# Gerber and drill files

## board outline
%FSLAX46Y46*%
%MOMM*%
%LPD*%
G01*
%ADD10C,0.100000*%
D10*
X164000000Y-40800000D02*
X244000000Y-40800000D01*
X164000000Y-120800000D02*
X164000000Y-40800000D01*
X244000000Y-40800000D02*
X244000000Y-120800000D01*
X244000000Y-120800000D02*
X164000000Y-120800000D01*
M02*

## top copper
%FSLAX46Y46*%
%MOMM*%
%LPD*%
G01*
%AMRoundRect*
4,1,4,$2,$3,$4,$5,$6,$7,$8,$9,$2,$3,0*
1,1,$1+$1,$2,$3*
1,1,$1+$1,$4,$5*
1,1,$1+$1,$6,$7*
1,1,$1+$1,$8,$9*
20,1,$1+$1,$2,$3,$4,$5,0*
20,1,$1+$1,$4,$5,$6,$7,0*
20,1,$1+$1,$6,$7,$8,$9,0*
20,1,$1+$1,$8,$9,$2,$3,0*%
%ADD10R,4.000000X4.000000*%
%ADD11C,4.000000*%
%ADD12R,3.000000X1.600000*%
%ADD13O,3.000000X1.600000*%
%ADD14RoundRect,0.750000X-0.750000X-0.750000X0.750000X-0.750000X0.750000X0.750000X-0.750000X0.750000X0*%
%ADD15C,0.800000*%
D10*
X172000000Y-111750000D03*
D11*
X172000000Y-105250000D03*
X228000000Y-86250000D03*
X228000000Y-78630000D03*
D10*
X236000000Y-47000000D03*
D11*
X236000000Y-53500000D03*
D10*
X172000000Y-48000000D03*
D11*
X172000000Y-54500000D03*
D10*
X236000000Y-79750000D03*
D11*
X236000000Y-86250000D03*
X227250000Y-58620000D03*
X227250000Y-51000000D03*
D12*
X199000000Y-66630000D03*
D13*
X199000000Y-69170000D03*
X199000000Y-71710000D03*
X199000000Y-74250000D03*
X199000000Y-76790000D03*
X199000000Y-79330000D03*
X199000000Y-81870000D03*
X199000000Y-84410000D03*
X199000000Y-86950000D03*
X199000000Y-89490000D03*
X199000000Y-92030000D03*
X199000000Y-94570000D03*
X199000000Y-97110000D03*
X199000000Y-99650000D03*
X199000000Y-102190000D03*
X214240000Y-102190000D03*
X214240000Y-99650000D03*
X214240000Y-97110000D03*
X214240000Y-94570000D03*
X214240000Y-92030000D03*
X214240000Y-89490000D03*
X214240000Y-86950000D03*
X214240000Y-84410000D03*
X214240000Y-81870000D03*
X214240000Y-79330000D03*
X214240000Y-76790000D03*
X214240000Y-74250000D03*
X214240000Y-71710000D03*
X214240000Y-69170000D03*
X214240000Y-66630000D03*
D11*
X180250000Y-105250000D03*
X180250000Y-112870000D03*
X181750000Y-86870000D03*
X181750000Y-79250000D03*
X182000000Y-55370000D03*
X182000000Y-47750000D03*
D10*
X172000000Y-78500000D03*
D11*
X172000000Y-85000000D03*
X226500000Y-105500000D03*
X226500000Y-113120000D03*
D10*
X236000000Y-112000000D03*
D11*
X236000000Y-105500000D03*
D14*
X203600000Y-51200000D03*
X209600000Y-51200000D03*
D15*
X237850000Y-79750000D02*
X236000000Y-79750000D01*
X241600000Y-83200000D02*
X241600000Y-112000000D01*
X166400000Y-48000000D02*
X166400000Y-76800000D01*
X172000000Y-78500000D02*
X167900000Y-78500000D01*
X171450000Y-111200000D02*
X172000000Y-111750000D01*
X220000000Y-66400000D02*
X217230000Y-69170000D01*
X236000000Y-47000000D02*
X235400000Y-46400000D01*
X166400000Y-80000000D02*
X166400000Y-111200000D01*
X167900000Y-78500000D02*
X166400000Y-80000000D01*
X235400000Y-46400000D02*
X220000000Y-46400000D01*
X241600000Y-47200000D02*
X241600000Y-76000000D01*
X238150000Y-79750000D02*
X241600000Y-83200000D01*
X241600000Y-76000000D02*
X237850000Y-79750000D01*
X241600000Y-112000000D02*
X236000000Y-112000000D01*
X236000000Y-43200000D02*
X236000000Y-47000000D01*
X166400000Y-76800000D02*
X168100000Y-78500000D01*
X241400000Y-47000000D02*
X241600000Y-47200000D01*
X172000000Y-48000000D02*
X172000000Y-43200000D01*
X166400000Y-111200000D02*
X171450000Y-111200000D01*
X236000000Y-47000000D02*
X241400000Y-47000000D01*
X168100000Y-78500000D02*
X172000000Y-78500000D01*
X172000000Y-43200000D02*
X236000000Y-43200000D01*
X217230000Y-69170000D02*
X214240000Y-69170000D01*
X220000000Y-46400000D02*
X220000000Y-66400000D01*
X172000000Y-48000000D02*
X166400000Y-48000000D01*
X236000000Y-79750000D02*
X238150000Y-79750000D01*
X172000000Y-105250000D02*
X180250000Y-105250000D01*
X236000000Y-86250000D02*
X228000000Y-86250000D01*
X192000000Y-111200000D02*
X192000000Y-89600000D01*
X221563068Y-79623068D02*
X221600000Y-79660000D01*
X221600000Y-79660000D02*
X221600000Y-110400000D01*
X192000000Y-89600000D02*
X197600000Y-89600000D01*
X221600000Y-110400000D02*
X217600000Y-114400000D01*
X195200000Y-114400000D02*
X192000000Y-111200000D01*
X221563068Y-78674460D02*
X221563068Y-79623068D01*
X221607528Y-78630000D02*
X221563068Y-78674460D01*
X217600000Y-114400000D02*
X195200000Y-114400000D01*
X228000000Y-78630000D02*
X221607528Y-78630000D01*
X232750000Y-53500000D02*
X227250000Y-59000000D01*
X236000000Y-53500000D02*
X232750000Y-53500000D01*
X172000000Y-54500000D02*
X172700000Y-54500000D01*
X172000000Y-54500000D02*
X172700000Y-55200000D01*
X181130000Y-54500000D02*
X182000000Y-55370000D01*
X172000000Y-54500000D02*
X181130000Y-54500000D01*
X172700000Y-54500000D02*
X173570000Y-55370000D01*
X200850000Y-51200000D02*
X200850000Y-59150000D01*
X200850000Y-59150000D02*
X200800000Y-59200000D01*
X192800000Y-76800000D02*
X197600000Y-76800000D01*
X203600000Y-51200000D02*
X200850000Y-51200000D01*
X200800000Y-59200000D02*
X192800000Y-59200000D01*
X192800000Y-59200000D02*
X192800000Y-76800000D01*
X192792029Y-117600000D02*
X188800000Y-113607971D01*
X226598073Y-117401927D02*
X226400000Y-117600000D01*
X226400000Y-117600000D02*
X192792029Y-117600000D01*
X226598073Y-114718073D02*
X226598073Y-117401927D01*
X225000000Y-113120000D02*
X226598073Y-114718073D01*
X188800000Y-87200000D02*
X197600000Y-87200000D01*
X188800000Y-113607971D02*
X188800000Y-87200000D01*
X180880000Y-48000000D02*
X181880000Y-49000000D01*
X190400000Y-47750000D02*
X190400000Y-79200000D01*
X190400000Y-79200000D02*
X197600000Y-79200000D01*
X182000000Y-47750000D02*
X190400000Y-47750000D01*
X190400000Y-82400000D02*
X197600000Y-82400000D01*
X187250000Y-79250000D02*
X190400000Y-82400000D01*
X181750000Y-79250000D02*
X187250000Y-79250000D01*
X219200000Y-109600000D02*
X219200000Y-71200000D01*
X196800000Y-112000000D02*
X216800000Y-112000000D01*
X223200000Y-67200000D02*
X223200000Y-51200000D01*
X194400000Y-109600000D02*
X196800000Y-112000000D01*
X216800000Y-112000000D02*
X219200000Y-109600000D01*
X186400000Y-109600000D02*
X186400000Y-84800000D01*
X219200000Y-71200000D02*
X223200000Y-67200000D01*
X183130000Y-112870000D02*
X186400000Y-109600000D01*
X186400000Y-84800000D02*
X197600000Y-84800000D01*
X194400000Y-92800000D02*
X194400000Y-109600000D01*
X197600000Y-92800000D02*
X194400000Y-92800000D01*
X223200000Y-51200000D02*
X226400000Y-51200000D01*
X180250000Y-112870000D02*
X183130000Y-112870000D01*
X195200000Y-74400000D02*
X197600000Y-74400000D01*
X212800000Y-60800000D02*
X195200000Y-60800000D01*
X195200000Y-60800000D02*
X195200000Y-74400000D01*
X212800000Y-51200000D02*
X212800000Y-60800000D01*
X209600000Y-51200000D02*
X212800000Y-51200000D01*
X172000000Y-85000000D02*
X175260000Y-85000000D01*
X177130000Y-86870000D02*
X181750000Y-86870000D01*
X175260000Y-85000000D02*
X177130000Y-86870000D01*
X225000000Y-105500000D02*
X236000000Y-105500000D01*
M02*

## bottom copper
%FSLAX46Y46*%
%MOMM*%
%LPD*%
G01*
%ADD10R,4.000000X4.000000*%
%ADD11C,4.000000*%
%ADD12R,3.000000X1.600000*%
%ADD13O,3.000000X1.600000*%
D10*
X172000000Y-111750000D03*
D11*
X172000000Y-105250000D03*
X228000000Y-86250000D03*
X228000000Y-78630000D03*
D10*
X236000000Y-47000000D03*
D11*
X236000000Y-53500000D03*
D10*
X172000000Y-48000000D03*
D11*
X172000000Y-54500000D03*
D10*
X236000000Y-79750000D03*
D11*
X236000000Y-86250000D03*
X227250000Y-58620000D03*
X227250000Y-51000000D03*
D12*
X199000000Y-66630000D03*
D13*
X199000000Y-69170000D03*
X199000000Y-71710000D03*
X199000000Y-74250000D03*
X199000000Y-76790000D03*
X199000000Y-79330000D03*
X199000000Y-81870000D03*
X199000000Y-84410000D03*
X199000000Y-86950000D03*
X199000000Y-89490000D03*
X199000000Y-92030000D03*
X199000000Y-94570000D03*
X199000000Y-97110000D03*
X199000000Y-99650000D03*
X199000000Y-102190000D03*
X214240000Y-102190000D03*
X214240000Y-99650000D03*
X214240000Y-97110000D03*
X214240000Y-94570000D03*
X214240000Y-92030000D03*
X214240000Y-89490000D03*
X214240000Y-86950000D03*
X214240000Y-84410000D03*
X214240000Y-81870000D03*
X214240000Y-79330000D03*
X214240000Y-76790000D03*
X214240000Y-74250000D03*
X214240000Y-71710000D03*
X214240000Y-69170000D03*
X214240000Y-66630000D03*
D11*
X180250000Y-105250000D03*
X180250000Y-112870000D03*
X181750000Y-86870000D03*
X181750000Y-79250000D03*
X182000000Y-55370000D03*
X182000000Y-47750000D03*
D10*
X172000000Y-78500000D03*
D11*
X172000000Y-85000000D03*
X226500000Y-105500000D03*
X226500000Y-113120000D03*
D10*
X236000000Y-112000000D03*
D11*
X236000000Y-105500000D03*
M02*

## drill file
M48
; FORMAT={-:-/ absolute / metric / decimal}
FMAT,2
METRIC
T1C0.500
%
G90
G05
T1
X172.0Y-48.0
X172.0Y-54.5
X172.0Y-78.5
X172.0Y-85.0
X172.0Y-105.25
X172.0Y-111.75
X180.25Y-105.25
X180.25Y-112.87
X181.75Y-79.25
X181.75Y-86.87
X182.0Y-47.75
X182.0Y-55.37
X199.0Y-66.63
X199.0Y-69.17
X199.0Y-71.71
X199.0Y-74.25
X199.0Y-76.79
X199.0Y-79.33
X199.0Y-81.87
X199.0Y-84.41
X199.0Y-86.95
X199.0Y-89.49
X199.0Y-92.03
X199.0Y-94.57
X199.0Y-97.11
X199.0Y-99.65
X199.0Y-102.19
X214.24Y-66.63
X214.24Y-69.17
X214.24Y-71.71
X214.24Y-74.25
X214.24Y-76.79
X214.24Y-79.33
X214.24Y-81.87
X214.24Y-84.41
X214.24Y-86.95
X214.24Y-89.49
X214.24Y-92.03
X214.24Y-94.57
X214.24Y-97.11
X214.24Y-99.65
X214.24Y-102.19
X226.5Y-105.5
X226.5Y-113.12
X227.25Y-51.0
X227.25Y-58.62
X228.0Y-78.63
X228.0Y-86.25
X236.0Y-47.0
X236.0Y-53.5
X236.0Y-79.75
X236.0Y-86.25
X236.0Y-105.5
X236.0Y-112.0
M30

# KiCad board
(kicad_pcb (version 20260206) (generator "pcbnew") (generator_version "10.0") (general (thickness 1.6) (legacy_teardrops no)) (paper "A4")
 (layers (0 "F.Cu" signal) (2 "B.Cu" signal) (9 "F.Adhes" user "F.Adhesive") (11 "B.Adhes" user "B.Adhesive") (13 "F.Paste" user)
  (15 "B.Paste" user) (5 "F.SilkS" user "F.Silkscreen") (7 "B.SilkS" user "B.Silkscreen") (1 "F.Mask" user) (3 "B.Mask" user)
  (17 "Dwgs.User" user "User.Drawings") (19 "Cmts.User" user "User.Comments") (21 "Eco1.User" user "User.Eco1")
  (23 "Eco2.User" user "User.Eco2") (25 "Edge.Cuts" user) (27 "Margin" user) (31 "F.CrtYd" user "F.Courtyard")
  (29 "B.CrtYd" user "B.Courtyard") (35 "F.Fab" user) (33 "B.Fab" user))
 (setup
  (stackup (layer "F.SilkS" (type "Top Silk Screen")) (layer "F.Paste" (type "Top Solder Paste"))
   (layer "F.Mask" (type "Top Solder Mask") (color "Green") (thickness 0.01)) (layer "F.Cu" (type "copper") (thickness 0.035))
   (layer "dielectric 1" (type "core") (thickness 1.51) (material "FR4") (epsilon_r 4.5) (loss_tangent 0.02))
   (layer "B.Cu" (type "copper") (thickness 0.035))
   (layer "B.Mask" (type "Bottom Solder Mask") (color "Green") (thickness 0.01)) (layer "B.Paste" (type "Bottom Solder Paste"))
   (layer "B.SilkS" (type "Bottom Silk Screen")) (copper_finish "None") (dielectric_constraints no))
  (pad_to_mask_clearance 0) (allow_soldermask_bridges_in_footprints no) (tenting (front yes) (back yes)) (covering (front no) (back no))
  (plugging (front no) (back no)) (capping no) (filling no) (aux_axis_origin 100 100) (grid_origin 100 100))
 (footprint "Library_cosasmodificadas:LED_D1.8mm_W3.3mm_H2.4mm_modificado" (layer "F.Cu") (at 172 109.25 90)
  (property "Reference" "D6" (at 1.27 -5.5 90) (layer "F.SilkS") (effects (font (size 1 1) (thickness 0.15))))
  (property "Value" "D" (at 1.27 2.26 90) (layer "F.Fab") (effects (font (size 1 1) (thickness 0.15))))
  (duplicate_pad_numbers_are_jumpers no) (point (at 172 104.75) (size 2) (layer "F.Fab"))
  (pad "1" thru_hole rect (at -2.5 0 90) (size 4 4) (drill 0.5) (layers "*.Cu" "*.Mask") (remove_unused_layers no) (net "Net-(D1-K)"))
  (pad "2" thru_hole circle (at 4 0 90) (size 4 4) (drill 0.5) (layers "*.Cu" "*.Mask") (remove_unused_layers no) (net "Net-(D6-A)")))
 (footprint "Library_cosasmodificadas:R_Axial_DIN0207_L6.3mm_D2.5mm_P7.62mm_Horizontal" (layer "F.Cu") (at 228 86.25 90)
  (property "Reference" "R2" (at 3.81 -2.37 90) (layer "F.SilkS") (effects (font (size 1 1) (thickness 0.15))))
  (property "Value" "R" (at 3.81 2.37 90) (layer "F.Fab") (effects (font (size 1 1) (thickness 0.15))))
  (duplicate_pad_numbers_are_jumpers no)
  (pad "1" thru_hole circle (at 0 0 90) (size 4 4) (drill 0.5) (layers "*.Cu" "*.Mask") (remove_unused_layers no) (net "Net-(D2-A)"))
  (pad "2" thru_hole circle (at 7.62 0 90) (size 4 4) (drill 0.5) (layers "*.Cu" "*.Mask") (remove_unused_layers no) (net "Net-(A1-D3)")))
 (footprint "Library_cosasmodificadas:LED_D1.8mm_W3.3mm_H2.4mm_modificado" (layer "F.Cu") (at 236 49.5 -90)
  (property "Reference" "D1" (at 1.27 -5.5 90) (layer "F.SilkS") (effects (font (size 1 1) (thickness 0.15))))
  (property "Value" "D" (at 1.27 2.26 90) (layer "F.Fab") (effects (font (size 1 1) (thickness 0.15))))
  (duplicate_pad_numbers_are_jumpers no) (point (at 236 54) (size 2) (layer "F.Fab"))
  (pad "1" thru_hole rect (at -2.5 0 270) (size 4 4) (drill 0.5) (layers "*.Cu" "*.Mask") (remove_unused_layers no) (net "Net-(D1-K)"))
  (pad "2" thru_hole circle (at 4 0 270) (size 4 4) (drill 0.5) (layers "*.Cu" "*.Mask") (remove_unused_layers no) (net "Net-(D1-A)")))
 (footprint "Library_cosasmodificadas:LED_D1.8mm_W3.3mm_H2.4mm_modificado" (layer "F.Cu") (at 172 50.5 -90)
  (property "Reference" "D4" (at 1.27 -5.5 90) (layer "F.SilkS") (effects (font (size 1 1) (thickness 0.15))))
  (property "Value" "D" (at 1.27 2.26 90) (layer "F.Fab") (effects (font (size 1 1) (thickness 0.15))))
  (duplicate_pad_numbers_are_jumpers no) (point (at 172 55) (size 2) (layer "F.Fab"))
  (pad "1" thru_hole rect (at -2.5 0 270) (size 4 4) (drill 0.5) (layers "*.Cu" "*.Mask") (remove_unused_layers no) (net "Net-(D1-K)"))
  (pad "2" thru_hole circle (at 4 0 270) (size 4 4) (drill 0.5) (layers "*.Cu" "*.Mask") (remove_unused_layers no) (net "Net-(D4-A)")))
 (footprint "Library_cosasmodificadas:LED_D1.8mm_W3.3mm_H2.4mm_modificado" (layer "F.Cu") (at 236 82.25 -90)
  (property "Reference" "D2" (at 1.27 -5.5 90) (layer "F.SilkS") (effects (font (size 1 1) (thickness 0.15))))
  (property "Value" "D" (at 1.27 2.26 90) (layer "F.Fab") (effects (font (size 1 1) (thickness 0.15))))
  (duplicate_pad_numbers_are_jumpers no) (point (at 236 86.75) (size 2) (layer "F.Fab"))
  (pad "1" thru_hole rect (at -2.5 0 270) (size 4 4) (drill 0.5) (layers "*.Cu" "*.Mask") (remove_unused_layers no) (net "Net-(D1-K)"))
  (pad "2" thru_hole circle (at 4 0 270) (size 4 4) (drill 0.5) (layers "*.Cu" "*.Mask") (remove_unused_layers no) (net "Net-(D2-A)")))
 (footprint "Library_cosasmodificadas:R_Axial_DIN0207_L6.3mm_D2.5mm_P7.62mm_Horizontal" (layer "F.Cu") (at 227.25 58.62 90)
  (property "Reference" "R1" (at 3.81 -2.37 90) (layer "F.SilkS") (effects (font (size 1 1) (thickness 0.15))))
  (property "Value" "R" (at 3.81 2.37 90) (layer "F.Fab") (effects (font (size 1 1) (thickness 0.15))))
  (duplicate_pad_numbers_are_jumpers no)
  (pad "1" thru_hole circle (at 0 0 90) (size 4 4) (drill 0.5) (layers "*.Cu" "*.Mask") (remove_unused_layers no) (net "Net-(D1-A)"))
  (pad "2" thru_hole circle (at 7.62 0 90) (size 4 4) (drill 0.5) (layers "*.Cu" "*.Mask") (remove_unused_layers no) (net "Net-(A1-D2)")))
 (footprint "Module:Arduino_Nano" (layer "F.Cu") (at 199 66.63)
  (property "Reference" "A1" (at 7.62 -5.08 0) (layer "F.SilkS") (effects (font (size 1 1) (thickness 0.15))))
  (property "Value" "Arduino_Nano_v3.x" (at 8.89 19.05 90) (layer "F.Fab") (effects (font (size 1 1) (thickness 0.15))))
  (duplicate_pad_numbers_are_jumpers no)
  (pad "1" thru_hole rect (at 0 0) (size 3 1.6) (drill 0.5) (layers "*.Cu" "*.Mask") (remove_unused_layers no)
   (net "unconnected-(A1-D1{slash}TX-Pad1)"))
  (pad "2" thru_hole oval (at 0 2.54) (size 3 1.6) (drill 0.5) (layers "*.Cu" "*.Mask") (remove_unused_layers no)
   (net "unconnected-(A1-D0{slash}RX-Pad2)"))
  (pad "3" thru_hole oval (at 0 5.08) (size 3 1.6) (drill 0.5) (layers "*.Cu" "*.Mask") (remove_unused_layers no)
   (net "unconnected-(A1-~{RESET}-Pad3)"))
  (pad "4" thru_hole oval (at 0 7.62) (size 3 1.6) (drill 0.5) (layers "*.Cu" "*.Mask") (remove_unused_layers no) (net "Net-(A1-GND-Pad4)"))
  (pad "5" thru_hole oval (at 0 10.16) (size 3 1.6) (drill 0.5) (layers "*.Cu" "*.Mask") (remove_unused_layers no) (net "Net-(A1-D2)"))
  (pad "6" thru_hole oval (at 0 12.7) (size 3 1.6) (drill 0.5) (layers "*.Cu" "*.Mask") (remove_unused_layers no) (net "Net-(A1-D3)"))
  (pad "7" thru_hole oval (at 0 15.24) (size 3 1.6) (drill 0.5) (layers "*.Cu" "*.Mask") (remove_unused_layers no) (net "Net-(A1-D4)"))
  (pad "8" thru_hole oval (at 0 17.78) (size 3 1.6) (drill 0.5) (layers "*.Cu" "*.Mask") (remove_unused_layers no) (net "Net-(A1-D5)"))
  (pad "9" thru_hole oval (at 0 20.32) (size 3 1.6) (drill 0.5) (layers "*.Cu" "*.Mask") (remove_unused_layers no) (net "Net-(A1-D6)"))
  (pad "10" thru_hole oval (at 0 22.86) (size 3 1.6) (drill 0.5) (layers "*.Cu" "*.Mask") (remove_unused_layers no)
   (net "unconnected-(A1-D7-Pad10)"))
  (pad "11" thru_hole oval (at 0 25.4) (size 3 1.6) (drill 0.5) (layers "*.Cu" "*.Mask") (remove_unused_layers no) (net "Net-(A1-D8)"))
  (pad "12" thru_hole oval (at 0 27.94) (size 3 1.6) (drill 0.5) (layers "*.Cu" "*.Mask") (remove_unused_layers no)
   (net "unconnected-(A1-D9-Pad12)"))
  (pad "13" thru_hole oval (at 0 30.48) (size 3 1.6) (drill 0.5) (layers "*.Cu" "*.Mask") (remove_unused_layers no)
   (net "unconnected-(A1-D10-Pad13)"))
  (pad "14" thru_hole oval (at 0 33.02) (size 3 1.6) (drill 0.5) (layers "*.Cu" "*.Mask") (remove_unused_layers no)
   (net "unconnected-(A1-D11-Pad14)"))
  (pad "15" thru_hole oval (at 0 35.56) (size 3 1.6) (drill 0.5) (layers "*.Cu" "*.Mask") (remove_unused_layers no)
   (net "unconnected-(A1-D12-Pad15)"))
  (pad "16" thru_hole oval (at 15.24 35.56) (size 3 1.6) (drill 0.5) (layers "*.Cu" "*.Mask") (remove_unused_layers no) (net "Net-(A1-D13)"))
  (pad "17" thru_hole oval (at 15.24 33.02) (size 3 1.6) (drill 0.5) (layers "*.Cu" "*.Mask") (remove_unused_layers no)
   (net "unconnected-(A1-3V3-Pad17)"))
  (pad "18" thru_hole oval (at 15.24 30.48) (size 3 1.6) (drill 0.5) (layers "*.Cu" "*.Mask") (remove_unused_layers no)
   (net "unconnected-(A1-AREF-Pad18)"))
  (pad "19" thru_hole oval (at 15.24 27.94) (size 3 1.6) (drill 0.5) (layers "*.Cu" "*.Mask") (remove_unused_layers no)
   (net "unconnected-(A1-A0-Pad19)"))
  (pad "20" thru_hole oval (at 15.24 25.4) (size 3 1.6) (drill 0.5) (layers "*.Cu" "*.Mask") (remove_unused_layers no)
   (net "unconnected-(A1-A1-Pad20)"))
  (pad "21" thru_hole oval (at 15.24 22.86) (size 3 1.6) (drill 0.5) (layers "*.Cu" "*.Mask") (remove_unused_layers no)
   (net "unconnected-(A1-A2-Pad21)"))
  (pad "22" thru_hole oval (at 15.24 20.32) (size 3 1.6) (drill 0.5) (layers "*.Cu" "*.Mask") (remove_unused_layers no)
   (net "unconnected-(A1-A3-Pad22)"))
  (pad "23" thru_hole oval (at 15.24 17.78) (size 3 1.6) (drill 0.5) (layers "*.Cu" "*.Mask") (remove_unused_layers no)
   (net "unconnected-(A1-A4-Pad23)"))
  (pad "24" thru_hole oval (at 15.24 15.24) (size 3 1.6) (drill 0.5) (layers "*.Cu" "*.Mask") (remove_unused_layers no)
   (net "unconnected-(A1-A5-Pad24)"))
  (pad "25" thru_hole oval (at 15.24 12.7) (size 3 1.6) (drill 0.5) (layers "*.Cu" "*.Mask") (remove_unused_layers no)
   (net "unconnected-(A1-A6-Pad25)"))
  (pad "26" thru_hole oval (at 15.24 10.16) (size 3 1.6) (drill 0.5) (layers "*.Cu" "*.Mask") (remove_unused_layers no)
   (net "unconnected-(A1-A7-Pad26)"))
  (pad "27" thru_hole oval (at 15.24 7.62) (size 3 1.6) (drill 0.5) (layers "*.Cu" "*.Mask") (remove_unused_layers no)
   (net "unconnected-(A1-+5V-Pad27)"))
  (pad "28" thru_hole oval (at 15.24 5.08) (size 3 1.6) (drill 0.5) (layers "*.Cu" "*.Mask") (remove_unused_layers no)
   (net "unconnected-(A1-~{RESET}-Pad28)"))
  (pad "29" thru_hole oval (at 15.24 2.54) (size 3 1.6) (drill 0.5) (layers "*.Cu" "*.Mask") (remove_unused_layers no) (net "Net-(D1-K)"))
  (pad "30" thru_hole oval (at 15.24 0) (size 3 1.6) (drill 0.5) (layers "*.Cu" "*.Mask") (remove_unused_layers no)
   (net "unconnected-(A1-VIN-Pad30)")))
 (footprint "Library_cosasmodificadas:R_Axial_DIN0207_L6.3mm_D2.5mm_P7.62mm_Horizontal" (layer "F.Cu") (at 180.25 105.25 -90)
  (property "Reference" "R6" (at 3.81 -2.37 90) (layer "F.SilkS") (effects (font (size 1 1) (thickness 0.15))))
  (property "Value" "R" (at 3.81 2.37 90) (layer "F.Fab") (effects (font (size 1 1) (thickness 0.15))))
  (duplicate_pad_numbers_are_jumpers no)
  (pad "1" thru_hole circle (at 0 0 270) (size 4 4) (drill 0.5) (layers "*.Cu" "*.Mask") (remove_unused_layers no) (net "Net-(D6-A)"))
  (pad "2" thru_hole circle (at 7.62 0 270) (size 4 4) (drill 0.5) (layers "*.Cu" "*.Mask") (remove_unused_layers no) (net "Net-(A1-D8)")))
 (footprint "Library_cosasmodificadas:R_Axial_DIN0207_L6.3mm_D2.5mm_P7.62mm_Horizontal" (layer "F.Cu") (at 181.75 86.87 90)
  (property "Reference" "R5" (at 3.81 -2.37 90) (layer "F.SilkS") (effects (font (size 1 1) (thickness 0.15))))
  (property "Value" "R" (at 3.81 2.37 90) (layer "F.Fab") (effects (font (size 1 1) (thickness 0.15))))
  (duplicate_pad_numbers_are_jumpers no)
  (pad "1" thru_hole circle (at 0 0 90) (size 4 4) (drill 0.5) (layers "*.Cu" "*.Mask") (remove_unused_layers no) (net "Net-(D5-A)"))
  (pad "2" thru_hole circle (at 7.62 0 90) (size 4 4) (drill 0.5) (layers "*.Cu" "*.Mask") (remove_unused_layers no) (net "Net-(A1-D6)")))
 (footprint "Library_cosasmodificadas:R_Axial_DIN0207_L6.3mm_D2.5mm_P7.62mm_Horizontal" (layer "F.Cu") (at 182 55.37 90)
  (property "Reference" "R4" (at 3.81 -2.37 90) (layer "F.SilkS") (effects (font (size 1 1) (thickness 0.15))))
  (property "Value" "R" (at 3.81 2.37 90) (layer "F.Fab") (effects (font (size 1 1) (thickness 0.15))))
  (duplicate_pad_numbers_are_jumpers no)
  (pad "1" thru_hole circle (at 0 0 90) (size 4 4) (drill 0.5) (layers "*.Cu" "*.Mask") (remove_unused_layers no) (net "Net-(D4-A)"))
  (pad "2" thru_hole circle (at 7.62 0 90) (size 4 4) (drill 0.5) (layers "*.Cu" "*.Mask") (remove_unused_layers no) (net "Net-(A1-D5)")))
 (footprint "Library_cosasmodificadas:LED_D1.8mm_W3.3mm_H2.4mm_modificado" (layer "F.Cu") (at 172 81 -90)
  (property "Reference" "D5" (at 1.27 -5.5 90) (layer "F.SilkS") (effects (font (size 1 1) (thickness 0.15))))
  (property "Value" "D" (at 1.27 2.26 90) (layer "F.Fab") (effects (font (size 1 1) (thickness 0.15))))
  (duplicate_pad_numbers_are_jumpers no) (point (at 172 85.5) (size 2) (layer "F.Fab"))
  (pad "1" thru_hole rect (at -2.5 0 270) (size 4 4) (drill 0.5) (layers "*.Cu" "*.Mask") (remove_unused_layers no) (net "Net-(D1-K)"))
  (pad "2" thru_hole circle (at 4 0 270) (size 4 4) (drill 0.5) (layers "*.Cu" "*.Mask") (remove_unused_layers no) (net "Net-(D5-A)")))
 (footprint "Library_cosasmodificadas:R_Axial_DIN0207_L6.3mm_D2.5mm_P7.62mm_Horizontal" (layer "F.Cu") (at 226.5 105.5 -90)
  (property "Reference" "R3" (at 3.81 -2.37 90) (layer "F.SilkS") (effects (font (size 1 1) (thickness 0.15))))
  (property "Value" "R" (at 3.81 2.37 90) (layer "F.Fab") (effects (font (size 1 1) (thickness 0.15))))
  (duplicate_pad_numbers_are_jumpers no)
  (pad "1" thru_hole circle (at 0 0 270) (size 4 4) (drill 0.5) (layers "*.Cu" "*.Mask") (remove_unused_layers no) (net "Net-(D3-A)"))
  (pad "2" thru_hole circle (at 7.62 0 270) (size 4 4) (drill 0.5) (layers "*.Cu" "*.Mask") (remove_unused_layers no) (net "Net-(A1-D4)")))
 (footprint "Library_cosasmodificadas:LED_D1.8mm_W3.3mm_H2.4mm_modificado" (layer "F.Cu") (at 236 109.5 90)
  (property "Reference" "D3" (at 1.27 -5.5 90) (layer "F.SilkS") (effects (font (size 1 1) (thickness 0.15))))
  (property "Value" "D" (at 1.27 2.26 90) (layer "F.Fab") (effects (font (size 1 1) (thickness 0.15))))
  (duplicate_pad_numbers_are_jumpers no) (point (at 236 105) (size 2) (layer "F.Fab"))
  (pad "1" thru_hole rect (at -2.5 0 90) (size 4 4) (drill 0.5) (layers "*.Cu" "*.Mask") (remove_unused_layers no) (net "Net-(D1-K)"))
  (pad "2" thru_hole circle (at 4 0 90) (size 4 4) (drill 0.5) (layers "*.Cu" "*.Mask") (remove_unused_layers no) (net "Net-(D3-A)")))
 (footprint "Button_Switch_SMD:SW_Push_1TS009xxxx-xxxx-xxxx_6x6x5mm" (layer "F.Cu") (at 206.6 51.2)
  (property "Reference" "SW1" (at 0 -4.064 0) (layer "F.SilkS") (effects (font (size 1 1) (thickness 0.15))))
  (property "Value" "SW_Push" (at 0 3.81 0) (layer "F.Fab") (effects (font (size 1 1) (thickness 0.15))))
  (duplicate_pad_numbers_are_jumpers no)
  (pad "1" smd roundrect (at -3 0) (size 3 3) (layers "F.Cu" "F.Mask" "F.Paste") (roundrect_rratio 0.25) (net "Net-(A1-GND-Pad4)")
   (thermal_bridge_angle 45))
  (pad "2" smd roundrect (at 3 0) (size 3 3) (layers "F.Cu" "F.Mask" "F.Paste") (roundrect_rratio 0.25) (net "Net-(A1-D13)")
   (thermal_bridge_angle 45)))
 (gr_line (start 164 40.8) (end 244 40.8) (stroke (width 0.1) (type default)) (layer "Edge.Cuts"))
 (gr_line (start 164 120.8) (end 164 40.8) (stroke (width 0.1) (type default)) (layer "Edge.Cuts"))
 (gr_line (start 244 40.8) (end 244 120.8) (stroke (width 0.1) (type default)) (layer "Edge.Cuts"))
 (gr_line (start 244 120.8) (end 164 120.8) (stroke (width 0.1) (type default)) (layer "Edge.Cuts"))
 (segment (start 237.85 79.75) (end 236 79.75) (width 0.8) (layer "F.Cu") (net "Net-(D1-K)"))
 (segment (start 241.6 83.2) (end 241.6 112) (width 0.8) (layer "F.Cu") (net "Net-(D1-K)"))
 (segment (start 166.4 48) (end 166.4 76.8) (width 0.8) (layer "F.Cu") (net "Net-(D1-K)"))
 (segment (start 172 78.5) (end 167.9 78.5) (width 0.8) (layer "F.Cu") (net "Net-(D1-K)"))
 (segment (start 171.45 111.2) (end 172 111.75) (width 0.8) (layer "F.Cu") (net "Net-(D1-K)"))
 (segment (start 220 66.4) (end 217.23 69.17) (width 0.8) (layer "F.Cu") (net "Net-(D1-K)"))
 (segment (start 236 47) (end 235.4 46.4) (width 0.8) (layer "F.Cu") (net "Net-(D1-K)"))
 (segment (start 166.4 80) (end 166.4 111.2) (width 0.8) (layer "F.Cu") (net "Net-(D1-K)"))
 (segment (start 167.9 78.5) (end 166.4 80) (width 0.8) (layer "F.Cu") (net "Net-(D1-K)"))
 (segment (start 235.4 46.4) (end 220 46.4) (width 0.8) (layer "F.Cu") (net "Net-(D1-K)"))
 (segment (start 241.6 47.2) (end 241.6 76) (width 0.8) (layer "F.Cu") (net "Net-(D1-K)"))
 (segment (start 238.15 79.75) (end 241.6 83.2) (width 0.8) (layer "F.Cu") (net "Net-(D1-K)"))
 (segment (start 241.6 76) (end 237.85 79.75) (width 0.8) (layer "F.Cu") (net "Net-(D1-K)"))
 (segment (start 241.6 112) (end 236 112) (width 0.8) (layer "F.Cu") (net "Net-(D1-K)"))
 (segment (start 236 43.2) (end 236 47) (width 0.8) (layer "F.Cu") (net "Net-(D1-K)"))
 (segment (start 166.4 76.8) (end 168.1 78.5) (width 0.8) (layer "F.Cu") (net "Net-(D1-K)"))
 (segment (start 241.4 47) (end 241.6 47.2) (width 0.8) (layer "F.Cu") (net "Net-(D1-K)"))
 (segment (start 172 48) (end 172 43.2) (width 0.8) (layer "F.Cu") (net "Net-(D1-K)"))
 (segment (start 166.4 111.2) (end 171.45 111.2) (width 0.8) (layer "F.Cu") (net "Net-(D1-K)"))
 (segment (start 236 47) (end 241.4 47) (width 0.8) (layer "F.Cu") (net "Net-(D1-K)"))
 (segment (start 168.1 78.5) (end 172 78.5) (width 0.8) (layer "F.Cu") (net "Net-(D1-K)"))
 (segment (start 172 43.2) (end 236 43.2) (width 0.8) (layer "F.Cu") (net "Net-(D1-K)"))
 (segment (start 217.23 69.17) (end 214.24 69.17) (width 0.8) (layer "F.Cu") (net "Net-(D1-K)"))
 (segment (start 220 46.4) (end 220 66.4) (width 0.8) (layer "F.Cu") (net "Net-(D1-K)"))
 (segment (start 172 48) (end 166.4 48) (width 0.8) (layer "F.Cu") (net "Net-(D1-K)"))
 (segment (start 236 79.75) (end 238.15 79.75) (width 0.8) (layer "F.Cu") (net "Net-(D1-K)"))
 (segment (start 172 105.25) (end 180.25 105.25) (width 0.8) (layer "F.Cu") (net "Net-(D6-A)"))
 (segment (start 236 86.25) (end 228 86.25) (width 0.8) (layer "F.Cu") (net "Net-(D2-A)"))
 (segment (start 192 111.2) (end 192 89.6) (width 0.8) (layer "F.Cu") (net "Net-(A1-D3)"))
 (segment (start 221.563068 79.623068) (end 221.6 79.66) (width 0.8) (layer "F.Cu") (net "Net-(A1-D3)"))
 (segment (start 221.6 79.66) (end 221.6 110.4) (width 0.8) (layer "F.Cu") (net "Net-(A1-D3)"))
 (segment (start 192 89.6) (end 197.6 89.6) (width 0.8) (layer "F.Cu") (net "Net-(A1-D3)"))
 (segment (start 221.6 110.4) (end 217.6 114.4) (width 0.8) (layer "F.Cu") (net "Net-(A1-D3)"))
 (segment (start 195.2 114.4) (end 192 111.2) (width 0.8) (layer "F.Cu") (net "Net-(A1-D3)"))
 (segment (start 221.563068 78.67446) (end 221.563068 79.623068) (width 0.8) (layer "F.Cu") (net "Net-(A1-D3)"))
 (segment (start 221.607528 78.63) (end 221.563068 78.67446) (width 0.8) (layer "F.Cu") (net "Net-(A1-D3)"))
 (segment (start 217.6 114.4) (end 195.2 114.4) (width 0.8) (layer "F.Cu") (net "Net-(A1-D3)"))
 (segment (start 228 78.63) (end 221.607528 78.63) (width 0.8) (layer "F.Cu") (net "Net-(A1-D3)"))
 (segment (start 232.75 53.5) (end 227.25 59) (width 0.8) (layer "F.Cu") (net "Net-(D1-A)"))
 (segment (start 236 53.5) (end 232.75 53.5) (width 0.8) (layer "F.Cu") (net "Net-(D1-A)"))
 (segment (start 172 54.5) (end 172.7 54.5) (width 0.8) (layer "F.Cu") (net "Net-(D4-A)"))
 (segment (start 172 54.5) (end 172.7 55.2) (width 0.8) (layer "F.Cu") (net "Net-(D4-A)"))
 (segment (start 181.13 54.5) (end 182 55.37) (width 0.8) (layer "F.Cu") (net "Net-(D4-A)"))
 (segment (start 172 54.5) (end 181.13 54.5) (width 0.8) (layer "F.Cu") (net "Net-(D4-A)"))
 (segment (start 172.7 54.5) (end 173.57 55.37) (width 0.8) (layer "F.Cu") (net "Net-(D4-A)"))
 (segment (start 200.85 51.2) (end 200.85 59.15) (width 0.8) (layer "F.Cu") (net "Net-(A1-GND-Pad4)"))
 (segment (start 200.85 59.15) (end 200.8 59.2) (width 0.8) (layer "F.Cu") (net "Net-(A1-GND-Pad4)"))
 (segment (start 192.8 76.8) (end 197.6 76.8) (width 0.8) (layer "F.Cu") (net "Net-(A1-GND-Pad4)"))
 (segment (start 203.6 51.2) (end 200.85 51.2) (width 0.8) (layer "F.Cu") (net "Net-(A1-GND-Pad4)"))
 (segment (start 200.8 59.2) (end 192.8 59.2) (width 0.8) (layer "F.Cu") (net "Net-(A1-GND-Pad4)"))
 (segment (start 192.8 59.2) (end 192.8 76.8) (width 0.8) (layer "F.Cu") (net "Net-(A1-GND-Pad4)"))
 (segment (start 192.792029 117.6) (end 188.8 113.607971) (width 0.8) (layer "F.Cu") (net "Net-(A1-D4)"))
 (segment (start 226.598073 117.401927) (end 226.4 117.6) (width 0.8) (layer "F.Cu") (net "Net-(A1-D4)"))
 (segment (start 226.4 117.6) (end 192.792029 117.6) (width 0.8) (layer "F.Cu") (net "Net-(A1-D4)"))
 (segment (start 226.598073 114.718073) (end 226.598073 117.401927) (width 0.8) (layer "F.Cu") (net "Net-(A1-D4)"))
 (segment (start 225 113.12) (end 226.598073 114.718073) (width 0.8) (layer "F.Cu") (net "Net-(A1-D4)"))
 (segment (start 188.8 87.2) (end 197.6 87.2) (width 0.8) (layer "F.Cu") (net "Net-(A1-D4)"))
 (segment (start 188.8 113.607971) (end 188.8 87.2) (width 0.8) (layer "F.Cu") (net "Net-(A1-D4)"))
 (segment (start 180.88 48) (end 181.88 49) (width 0.8) (layer "F.Cu") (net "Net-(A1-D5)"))
 (segment (start 190.4 47.75) (end 190.4 79.2) (width 0.8) (layer "F.Cu") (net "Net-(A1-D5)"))
 (segment (start 190.4 79.2) (end 197.6 79.2) (width 0.8) (layer "F.Cu") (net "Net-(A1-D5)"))
 (segment (start 182 47.75) (end 190.4 47.75) (width 0.8) (layer "F.Cu") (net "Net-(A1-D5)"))
 (segment (start 190.4 82.4) (end 197.6 82.4) (width 0.8) (layer "F.Cu") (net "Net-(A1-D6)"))
 (segment (start 187.25 79.25) (end 190.4 82.4) (width 0.8) (layer "F.Cu") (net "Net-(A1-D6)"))
 (segment (start 181.75 79.25) (end 187.25 79.25) (width 0.8) (layer "F.Cu") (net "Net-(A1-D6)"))
 (segment (start 219.2 109.6) (end 219.2 71.2) (width 0.8) (layer "F.Cu") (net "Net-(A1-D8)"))
 (segment (start 196.8 112) (end 216.8 112) (width 0.8) (layer "F.Cu") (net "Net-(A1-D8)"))
 (segment (start 223.2 67.2) (end 223.2 51.2) (width 0.8) (layer "F.Cu") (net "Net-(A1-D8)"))
 (segment (start 194.4 109.6) (end 196.8 112) (width 0.8) (layer "F.Cu") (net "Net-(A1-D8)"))
 (segment (start 216.8 112) (end 219.2 109.6) (width 0.8) (layer "F.Cu") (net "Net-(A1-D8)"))
 (segment (start 186.4 109.6) (end 186.4 84.8) (width 0.8) (layer "F.Cu") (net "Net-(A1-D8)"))
 (segment (start 219.2 71.2) (end 223.2 67.2) (width 0.8) (layer "F.Cu") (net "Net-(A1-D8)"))
 (segment (start 183.13 112.87) (end 186.4 109.6) (width 0.8) (layer "F.Cu") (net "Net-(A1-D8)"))
 (segment (start 186.4 84.8) (end 197.6 84.8) (width 0.8) (layer "F.Cu") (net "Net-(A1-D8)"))
 (segment (start 194.4 92.8) (end 194.4 109.6) (width 0.8) (layer "F.Cu") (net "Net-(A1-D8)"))
 (segment (start 197.6 92.8) (end 194.4 92.8) (width 0.8) (layer "F.Cu") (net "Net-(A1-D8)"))
 (segment (start 223.2 51.2) (end 226.4 51.2) (width 0.8) (layer "F.Cu") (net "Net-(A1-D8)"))
 (segment (start 180.25 112.87) (end 183.13 112.87) (width 0.8) (layer "F.Cu") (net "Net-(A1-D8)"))
 (segment (start 195.2 74.4) (end 197.6 74.4) (width 0.8) (layer "F.Cu") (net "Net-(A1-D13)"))
 (segment (start 212.8 60.8) (end 195.2 60.8) (width 0.8) (layer "F.Cu") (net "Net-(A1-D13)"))
 (segment (start 195.2 60.8) (end 195.2 74.4) (width 0.8) (layer "F.Cu") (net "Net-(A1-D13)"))
 (segment (start 212.8 51.2) (end 212.8 60.8) (width 0.8) (layer "F.Cu") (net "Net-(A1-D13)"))
 (segment (start 209.6 51.2) (end 212.8 51.2) (width 0.8) (layer "F.Cu") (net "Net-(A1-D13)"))
 (segment (start 172 85) (end 175.26 85) (width 0.8) (layer "F.Cu") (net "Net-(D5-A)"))
 (segment (start 177.13 86.87) (end 181.75 86.87) (width 0.8) (layer "F.Cu") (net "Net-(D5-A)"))
 (segment (start 175.26 85) (end 177.13 86.87) (width 0.8) (layer "F.Cu") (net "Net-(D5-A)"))
 (segment (start 225 105.5) (end 236 105.5) (width 0.8) (layer "F.Cu") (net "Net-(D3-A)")))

